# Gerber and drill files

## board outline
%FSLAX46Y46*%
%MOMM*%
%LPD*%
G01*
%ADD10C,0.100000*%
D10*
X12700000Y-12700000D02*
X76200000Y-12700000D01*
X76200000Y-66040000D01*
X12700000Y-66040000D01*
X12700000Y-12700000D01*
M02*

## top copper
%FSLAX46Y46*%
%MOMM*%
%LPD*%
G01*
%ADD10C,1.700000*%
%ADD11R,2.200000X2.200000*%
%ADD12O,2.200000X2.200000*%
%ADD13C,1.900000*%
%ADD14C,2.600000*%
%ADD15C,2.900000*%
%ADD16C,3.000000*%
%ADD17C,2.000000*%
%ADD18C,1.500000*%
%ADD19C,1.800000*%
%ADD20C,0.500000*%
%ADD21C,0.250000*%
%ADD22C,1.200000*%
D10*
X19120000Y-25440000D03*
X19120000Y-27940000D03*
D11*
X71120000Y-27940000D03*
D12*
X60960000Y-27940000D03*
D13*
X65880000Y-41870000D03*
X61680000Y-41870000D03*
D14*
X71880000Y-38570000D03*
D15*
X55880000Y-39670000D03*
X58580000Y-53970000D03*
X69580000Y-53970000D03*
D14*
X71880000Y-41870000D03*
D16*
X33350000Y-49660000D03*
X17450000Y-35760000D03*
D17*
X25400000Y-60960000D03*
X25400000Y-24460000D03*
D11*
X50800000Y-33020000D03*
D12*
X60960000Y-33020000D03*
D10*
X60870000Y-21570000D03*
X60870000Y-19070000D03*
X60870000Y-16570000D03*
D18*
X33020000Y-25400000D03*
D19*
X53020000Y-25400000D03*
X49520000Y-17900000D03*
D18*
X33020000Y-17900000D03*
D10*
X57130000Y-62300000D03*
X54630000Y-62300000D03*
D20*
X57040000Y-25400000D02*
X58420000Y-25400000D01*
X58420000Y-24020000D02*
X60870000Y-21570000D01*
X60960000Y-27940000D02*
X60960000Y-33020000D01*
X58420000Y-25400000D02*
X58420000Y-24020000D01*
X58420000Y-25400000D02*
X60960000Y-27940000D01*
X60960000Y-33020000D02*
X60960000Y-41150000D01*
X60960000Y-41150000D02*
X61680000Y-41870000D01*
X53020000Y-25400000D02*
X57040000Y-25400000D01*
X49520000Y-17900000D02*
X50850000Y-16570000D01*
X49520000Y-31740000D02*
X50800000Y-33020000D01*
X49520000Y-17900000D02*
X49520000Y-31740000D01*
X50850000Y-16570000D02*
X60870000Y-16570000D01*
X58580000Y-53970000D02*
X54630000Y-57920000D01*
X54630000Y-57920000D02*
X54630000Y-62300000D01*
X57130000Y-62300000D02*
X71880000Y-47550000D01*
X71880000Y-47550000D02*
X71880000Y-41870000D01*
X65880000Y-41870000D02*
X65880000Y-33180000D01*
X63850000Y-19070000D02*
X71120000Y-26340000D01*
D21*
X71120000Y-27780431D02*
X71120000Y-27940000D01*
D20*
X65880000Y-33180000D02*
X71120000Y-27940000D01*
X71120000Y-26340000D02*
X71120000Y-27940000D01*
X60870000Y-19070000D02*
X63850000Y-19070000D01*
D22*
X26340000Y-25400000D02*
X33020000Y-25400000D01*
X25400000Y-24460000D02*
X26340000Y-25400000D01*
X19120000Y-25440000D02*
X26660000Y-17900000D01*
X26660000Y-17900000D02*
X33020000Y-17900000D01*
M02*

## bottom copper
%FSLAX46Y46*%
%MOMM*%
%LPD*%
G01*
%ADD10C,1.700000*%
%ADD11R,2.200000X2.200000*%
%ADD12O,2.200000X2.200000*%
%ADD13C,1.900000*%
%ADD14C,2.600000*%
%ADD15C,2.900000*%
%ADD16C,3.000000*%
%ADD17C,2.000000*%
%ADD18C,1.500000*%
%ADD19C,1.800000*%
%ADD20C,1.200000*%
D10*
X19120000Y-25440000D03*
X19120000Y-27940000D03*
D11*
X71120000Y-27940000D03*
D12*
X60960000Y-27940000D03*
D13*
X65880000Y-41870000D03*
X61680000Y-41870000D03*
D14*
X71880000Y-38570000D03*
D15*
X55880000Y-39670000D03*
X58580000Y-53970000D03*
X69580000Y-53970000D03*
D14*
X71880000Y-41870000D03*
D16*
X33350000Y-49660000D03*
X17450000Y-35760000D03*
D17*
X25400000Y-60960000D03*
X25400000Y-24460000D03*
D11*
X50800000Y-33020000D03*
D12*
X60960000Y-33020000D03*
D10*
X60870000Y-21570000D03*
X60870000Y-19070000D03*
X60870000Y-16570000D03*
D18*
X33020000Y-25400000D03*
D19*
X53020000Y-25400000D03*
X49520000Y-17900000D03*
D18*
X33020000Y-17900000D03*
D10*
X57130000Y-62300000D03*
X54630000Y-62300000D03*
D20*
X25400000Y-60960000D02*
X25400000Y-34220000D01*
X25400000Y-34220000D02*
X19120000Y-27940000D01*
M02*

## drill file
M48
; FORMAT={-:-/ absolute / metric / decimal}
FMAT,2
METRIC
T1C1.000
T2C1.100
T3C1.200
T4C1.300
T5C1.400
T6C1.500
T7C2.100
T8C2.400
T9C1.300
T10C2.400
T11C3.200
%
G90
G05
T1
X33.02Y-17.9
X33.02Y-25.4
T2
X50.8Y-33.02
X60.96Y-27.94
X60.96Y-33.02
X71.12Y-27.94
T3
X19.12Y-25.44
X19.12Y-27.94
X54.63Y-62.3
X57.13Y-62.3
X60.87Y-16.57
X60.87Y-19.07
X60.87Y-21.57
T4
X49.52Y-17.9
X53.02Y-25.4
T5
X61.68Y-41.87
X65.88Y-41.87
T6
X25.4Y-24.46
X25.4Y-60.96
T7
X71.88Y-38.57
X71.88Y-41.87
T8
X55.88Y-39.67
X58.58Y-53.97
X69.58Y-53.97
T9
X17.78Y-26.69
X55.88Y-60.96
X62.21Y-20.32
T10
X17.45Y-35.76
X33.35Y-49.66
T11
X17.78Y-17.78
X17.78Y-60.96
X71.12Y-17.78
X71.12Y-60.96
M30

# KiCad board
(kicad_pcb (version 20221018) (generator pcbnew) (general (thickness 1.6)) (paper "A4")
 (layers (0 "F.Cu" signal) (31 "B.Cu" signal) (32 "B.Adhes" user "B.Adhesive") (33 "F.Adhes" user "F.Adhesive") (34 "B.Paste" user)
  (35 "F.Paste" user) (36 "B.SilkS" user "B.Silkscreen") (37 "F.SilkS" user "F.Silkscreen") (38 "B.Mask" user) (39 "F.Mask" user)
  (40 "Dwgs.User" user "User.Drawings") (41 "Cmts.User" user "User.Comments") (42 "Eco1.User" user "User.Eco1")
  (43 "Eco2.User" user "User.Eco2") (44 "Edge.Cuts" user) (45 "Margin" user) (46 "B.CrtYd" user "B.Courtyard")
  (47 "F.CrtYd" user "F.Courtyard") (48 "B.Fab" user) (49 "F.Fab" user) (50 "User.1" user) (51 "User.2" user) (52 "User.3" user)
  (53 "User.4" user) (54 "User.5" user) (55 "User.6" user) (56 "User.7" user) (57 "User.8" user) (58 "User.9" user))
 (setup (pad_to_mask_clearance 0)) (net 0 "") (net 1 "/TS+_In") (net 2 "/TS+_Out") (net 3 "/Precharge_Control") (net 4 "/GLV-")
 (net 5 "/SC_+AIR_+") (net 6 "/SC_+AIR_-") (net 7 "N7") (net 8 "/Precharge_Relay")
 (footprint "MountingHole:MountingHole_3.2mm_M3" (layer "F.Cu") (at 71.12 17.78)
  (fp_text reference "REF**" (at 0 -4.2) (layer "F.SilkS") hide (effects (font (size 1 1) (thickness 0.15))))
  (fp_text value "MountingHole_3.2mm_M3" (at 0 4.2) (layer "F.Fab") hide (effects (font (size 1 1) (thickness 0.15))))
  (pad "" np_thru_hole circle (at 0 0) (size 3.2 3.2) (drill 3.2) (layers "*.Cu" "*.Mask")))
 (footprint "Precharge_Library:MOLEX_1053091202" (layer "F.Cu") (at 19.12 25.44 -90)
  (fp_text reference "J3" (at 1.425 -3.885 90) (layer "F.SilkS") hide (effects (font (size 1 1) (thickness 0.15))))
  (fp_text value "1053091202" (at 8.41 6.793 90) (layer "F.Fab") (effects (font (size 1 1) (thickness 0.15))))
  (pad "" np_thru_hole circle (at 1.25 1.34 270) (size 1.3 1.3) (drill 1.3) (layers "*.Cu" "*.Mask"))
  (pad "1" thru_hole circle (at 0 0 270) (size 1.7 1.7) (drill 1.2) (layers "*.Cu") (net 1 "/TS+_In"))
  (pad "2" thru_hole circle (at 2.5 0 270) (size 1.7 1.7) (drill 1.2) (layers "*.Cu") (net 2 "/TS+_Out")))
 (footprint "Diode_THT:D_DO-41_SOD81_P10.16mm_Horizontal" (layer "F.Cu") (at 71.12 27.94 180)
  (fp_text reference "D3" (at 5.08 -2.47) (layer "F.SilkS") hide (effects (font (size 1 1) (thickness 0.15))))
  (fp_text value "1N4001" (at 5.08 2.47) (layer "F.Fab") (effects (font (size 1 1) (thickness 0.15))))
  (pad "1" thru_hole rect (at 0 0 180) (size 2.2 2.2) (drill 1.1) (layers "*.Cu" "*.Mask") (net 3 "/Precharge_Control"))
  (pad "2" thru_hole oval (at 10.16 0 180) (size 2.2 2.2) (drill 1.1) (layers "*.Cu" "*.Mask") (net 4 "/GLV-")))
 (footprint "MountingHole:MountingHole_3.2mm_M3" (layer "F.Cu") (at 17.78 17.78)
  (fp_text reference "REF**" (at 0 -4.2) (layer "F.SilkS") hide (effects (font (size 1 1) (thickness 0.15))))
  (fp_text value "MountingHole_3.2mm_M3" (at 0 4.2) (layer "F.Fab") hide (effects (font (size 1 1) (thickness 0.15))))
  (pad "" np_thru_hole circle (at 0 0) (size 3.2 3.2) (drill 3.2) (layers "F&B.Cu" "*.Mask")))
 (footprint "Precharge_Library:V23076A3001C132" (layer "F.Cu") (at 49.18 35.27)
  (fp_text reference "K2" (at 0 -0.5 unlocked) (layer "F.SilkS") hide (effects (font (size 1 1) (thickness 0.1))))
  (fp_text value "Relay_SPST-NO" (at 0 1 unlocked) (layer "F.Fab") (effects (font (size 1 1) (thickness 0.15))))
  (pad "1" thru_hole circle (at 16.7 6.6) (size 1.9 1.9) (drill 1.4) (layers "*.Cu" "*.Mask") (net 3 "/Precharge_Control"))
  (pad "2" thru_hole circle (at 12.5 6.6) (size 1.9 1.9) (drill 1.4) (layers "*.Cu" "*.Mask") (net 4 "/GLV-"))
  (pad "3" thru_hole circle (at 22.7 3.3) (size 2.6 2.6) (drill 2.1) (layers "*.Cu" "*.Mask"))
  (pad "4" thru_hole circle (at 6.7 4.4) (size 2.9 2.9) (drill 2.4) (layers "*.Cu" "*.Mask") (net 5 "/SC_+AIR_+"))
  (pad "4" thru_hole circle (at 9.4 18.7) (size 2.9 2.9) (drill 2.4) (layers "*.Cu" "*.Mask") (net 5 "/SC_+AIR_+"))
  (pad "4" thru_hole circle (at 20.4 18.7) (size 2.9 2.9) (drill 2.4) (layers "*.Cu" "*.Mask") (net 5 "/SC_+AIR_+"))
  (pad "5" thru_hole circle (at 22.7 6.6) (size 2.6 2.6) (drill 2.1) (layers "*.Cu" "*.Mask") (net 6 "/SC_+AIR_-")))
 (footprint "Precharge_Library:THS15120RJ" (layer "F.Cu") (at 14.9 53.21 90)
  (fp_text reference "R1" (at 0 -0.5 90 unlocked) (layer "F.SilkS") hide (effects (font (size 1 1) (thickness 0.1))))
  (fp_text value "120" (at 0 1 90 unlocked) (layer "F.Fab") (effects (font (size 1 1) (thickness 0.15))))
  (pad "" np_thru_hole circle (at 3.55 18.45 90) (size 3 3) (drill 2.4) (layers "F&B.Cu" "*.Mask"))
  (pad "" np_thru_hole circle (at 17.45 2.55 90) (size 3 3) (drill 2.4) (layers "F&B.Cu" "*.Mask"))
  (pad "+" thru_hole circle (at -7.75 10.5 90) (size 2 2) (drill 1.5) (layers "*.Cu" "*.Mask") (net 2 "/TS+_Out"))
  (pad "-" thru_hole circle (at 28.75 10.5 90) (size 2 2) (drill 1.5) (layers "*.Cu" "*.Mask") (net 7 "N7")))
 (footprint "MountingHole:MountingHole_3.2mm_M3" (layer "F.Cu") (at 71.12 60.96)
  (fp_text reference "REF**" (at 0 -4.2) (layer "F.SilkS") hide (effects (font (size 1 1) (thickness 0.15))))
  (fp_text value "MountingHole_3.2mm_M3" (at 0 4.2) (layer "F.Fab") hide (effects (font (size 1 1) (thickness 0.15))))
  (pad "" np_thru_hole circle (at 0 0) (size 3.2 3.2) (drill 3.2) (layers "F&B.Cu" "*.Mask")))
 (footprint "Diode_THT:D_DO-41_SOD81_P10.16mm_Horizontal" (layer "F.Cu") (at 50.8 33.02)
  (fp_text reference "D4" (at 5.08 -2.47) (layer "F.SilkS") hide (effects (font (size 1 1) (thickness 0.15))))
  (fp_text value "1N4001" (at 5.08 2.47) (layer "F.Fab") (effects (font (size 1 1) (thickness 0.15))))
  (pad "1" thru_hole rect (at 0 0) (size 2.2 2.2) (drill 1.1) (layers "*.Cu" "*.Mask") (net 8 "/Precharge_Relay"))
  (pad "2" thru_hole oval (at 10.16 0) (size 2.2 2.2) (drill 1.1) (layers "*.Cu" "*.Mask") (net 4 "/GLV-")))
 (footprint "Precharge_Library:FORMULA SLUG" (layer "F.Cu") (at 65.44258 62.288544)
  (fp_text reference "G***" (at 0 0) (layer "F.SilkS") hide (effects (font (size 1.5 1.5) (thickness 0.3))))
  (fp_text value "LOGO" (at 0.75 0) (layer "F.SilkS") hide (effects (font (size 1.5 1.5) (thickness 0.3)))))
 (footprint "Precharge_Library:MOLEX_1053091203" (layer "F.Cu") (at 60.87 21.57 90)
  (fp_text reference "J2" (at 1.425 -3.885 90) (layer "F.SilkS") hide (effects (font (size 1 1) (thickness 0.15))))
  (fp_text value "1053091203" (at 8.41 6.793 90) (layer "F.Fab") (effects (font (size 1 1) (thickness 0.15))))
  (pad "" np_thru_hole circle (at 1.25 1.34 90) (size 1.3 1.3) (drill 1.3) (layers "*.Cu" "*.Mask"))
  (pad "1" thru_hole circle (at 0 0 90) (size 1.7 1.7) (drill 1.2) (layers "*.Cu") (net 4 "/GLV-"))
  (pad "2" thru_hole circle (at 2.5 0 90) (size 1.7 1.7) (drill 1.2) (layers "*.Cu") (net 3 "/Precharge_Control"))
  (pad "3" thru_hole circle (at 5 0 90) (size 1.7 1.7) (drill 1.2) (layers "*.Cu") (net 8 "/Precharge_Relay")))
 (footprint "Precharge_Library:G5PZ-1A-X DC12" (layer "F.Cu") (at 30.48 14.06)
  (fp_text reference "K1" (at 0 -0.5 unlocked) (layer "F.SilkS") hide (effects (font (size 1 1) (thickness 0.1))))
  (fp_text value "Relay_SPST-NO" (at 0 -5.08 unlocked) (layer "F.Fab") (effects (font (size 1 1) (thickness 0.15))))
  (pad "1" thru_hole circle (at 2.54 11.34) (size 1.5 1.5) (drill 1) (layers "*.Cu" "*.Mask") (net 7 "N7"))
  (pad "2" thru_hole circle (at 22.54 11.34) (size 1.8 1.8) (drill 1.3) (layers "*.Cu" "*.Mask") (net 4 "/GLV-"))
  (pad "3" thru_hole circle (at 19.04 3.84) (size 1.8 1.8) (drill 1.3) (layers "*.Cu" "*.Mask") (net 8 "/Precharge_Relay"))
  (pad "4" thru_hole circle (at 2.54 3.84) (size 1.5 1.5) (drill 1) (layers "*.Cu" "*.Mask") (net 1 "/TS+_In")))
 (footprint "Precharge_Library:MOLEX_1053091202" (layer "F.Cu") (at 57.13 62.3 180)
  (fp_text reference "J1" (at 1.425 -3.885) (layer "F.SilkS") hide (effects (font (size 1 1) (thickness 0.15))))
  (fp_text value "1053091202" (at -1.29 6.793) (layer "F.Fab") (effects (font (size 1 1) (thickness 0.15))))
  (pad "" np_thru_hole circle (at 1.25 1.34 180) (size 1.3 1.3) (drill 1.3) (layers "*.Cu" "*.Mask"))
  (pad "1" thru_hole circle (at 0 0 180) (size 1.7 1.7) (drill 1.2) (layers "*.Cu") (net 6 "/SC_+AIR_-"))
  (pad "2" thru_hole circle (at 2.5 0 180) (size 1.7 1.7) (drill 1.2) (layers "*.Cu") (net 5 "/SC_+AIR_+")))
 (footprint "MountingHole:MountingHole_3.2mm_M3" (layer "F.Cu") (at 17.78 60.96)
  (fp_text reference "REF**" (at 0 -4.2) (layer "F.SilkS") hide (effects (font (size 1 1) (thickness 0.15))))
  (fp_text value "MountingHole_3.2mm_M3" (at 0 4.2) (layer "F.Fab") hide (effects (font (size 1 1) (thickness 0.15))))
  (pad "" np_thru_hole circle (at 0 0) (size 3.2 3.2) (drill 3.2) (layers "F&B.Cu" "*.Mask")))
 (gr_rect (start 12.7 12.7) (end 76.2 66.04) (stroke (width 0.1) (type default)) (fill none) (layer "Edge.Cuts"))
 (segment (start 57.04 25.4) (end 58.42 25.4) (width 0.5) (layer "F.Cu") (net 4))
 (segment (start 58.42 24.02) (end 60.87 21.57) (width 0.5) (layer "F.Cu") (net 4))
 (segment (start 60.96 27.94) (end 60.96 33.02) (width 0.5) (layer "F.Cu") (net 4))
 (segment (start 58.42 25.4) (end 58.42 24.02) (width 0.5) (layer "F.Cu") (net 4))
 (segment (start 58.42 25.4) (end 60.96 27.94) (width 0.5) (layer "F.Cu") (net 4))
 (segment (start 60.96 33.02) (end 60.96 41.15) (width 0.5) (layer "F.Cu") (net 4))
 (segment (start 60.96 41.15) (end 61.68 41.87) (width 0.5) (layer "F.Cu") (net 4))
 (segment (start 53.02 25.4) (end 57.04 25.4) (width 0.5) (layer "F.Cu") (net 4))
 (segment (start 49.52 17.9) (end 50.85 16.57) (width 0.5) (layer "F.Cu") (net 8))
 (segment (start 49.52 31.74) (end 50.8 33.02) (width 0.5) (layer "F.Cu") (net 8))
 (segment (start 49.52 17.9) (end 49.52 31.74) (width 0.5) (layer "F.Cu") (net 8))
 (segment (start 50.85 16.57) (end 60.87 16.57) (width 0.5) (layer "F.Cu") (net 8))
 (segment (start 58.58 53.97) (end 54.63 57.92) (width 0.5) (layer "F.Cu") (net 5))
 (segment (start 54.63 57.92) (end 54.63 62.3) (width 0.5) (layer "F.Cu") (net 5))
 (segment (start 57.13 62.3) (end 71.88 47.55) (width 0.5) (layer "F.Cu") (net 6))
 (segment (start 71.88 47.55) (end 71.88 41.87) (width 0.5) (layer "F.Cu") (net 6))
 (segment (start 65.88 41.87) (end 65.88 33.18) (width 0.5) (layer "F.Cu") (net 3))
 (segment (start 63.85 19.07) (end 71.12 26.34) (width 0.5) (layer "F.Cu") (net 3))
 (segment (start 71.12 27.780431) (end 71.12 27.94) (width 0.25) (layer "F.Cu") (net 3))
 (segment (start 65.88 33.18) (end 71.12 27.94) (width 0.5) (layer "F.Cu") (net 3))
 (segment (start 71.12 26.34) (end 71.12 27.94) (width 0.5) (layer "F.Cu") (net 3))
 (segment (start 60.87 19.07) (end 63.85 19.07) (width 0.5) (layer "F.Cu") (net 3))
 (segment (start 25.4 60.96) (end 25.4 34.22) (width 1.2) (layer "B.Cu") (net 2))
 (segment (start 25.4 34.22) (end 19.12 27.94) (width 1.2) (layer "B.Cu") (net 2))
 (segment (start 26.34 25.4) (end 33.02 25.4) (width 1.2) (layer "F.Cu") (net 7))
 (segment (start 25.4 24.46) (end 26.34 25.4) (width 1.2) (layer "F.Cu") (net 7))
 (segment (start 19.12 25.44) (end 26.66 17.9) (width 1.2) (layer "F.Cu") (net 1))
 (segment (start 26.66 17.9) (end 33.02 17.9) (width 1.2) (layer "F.Cu") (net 1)))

